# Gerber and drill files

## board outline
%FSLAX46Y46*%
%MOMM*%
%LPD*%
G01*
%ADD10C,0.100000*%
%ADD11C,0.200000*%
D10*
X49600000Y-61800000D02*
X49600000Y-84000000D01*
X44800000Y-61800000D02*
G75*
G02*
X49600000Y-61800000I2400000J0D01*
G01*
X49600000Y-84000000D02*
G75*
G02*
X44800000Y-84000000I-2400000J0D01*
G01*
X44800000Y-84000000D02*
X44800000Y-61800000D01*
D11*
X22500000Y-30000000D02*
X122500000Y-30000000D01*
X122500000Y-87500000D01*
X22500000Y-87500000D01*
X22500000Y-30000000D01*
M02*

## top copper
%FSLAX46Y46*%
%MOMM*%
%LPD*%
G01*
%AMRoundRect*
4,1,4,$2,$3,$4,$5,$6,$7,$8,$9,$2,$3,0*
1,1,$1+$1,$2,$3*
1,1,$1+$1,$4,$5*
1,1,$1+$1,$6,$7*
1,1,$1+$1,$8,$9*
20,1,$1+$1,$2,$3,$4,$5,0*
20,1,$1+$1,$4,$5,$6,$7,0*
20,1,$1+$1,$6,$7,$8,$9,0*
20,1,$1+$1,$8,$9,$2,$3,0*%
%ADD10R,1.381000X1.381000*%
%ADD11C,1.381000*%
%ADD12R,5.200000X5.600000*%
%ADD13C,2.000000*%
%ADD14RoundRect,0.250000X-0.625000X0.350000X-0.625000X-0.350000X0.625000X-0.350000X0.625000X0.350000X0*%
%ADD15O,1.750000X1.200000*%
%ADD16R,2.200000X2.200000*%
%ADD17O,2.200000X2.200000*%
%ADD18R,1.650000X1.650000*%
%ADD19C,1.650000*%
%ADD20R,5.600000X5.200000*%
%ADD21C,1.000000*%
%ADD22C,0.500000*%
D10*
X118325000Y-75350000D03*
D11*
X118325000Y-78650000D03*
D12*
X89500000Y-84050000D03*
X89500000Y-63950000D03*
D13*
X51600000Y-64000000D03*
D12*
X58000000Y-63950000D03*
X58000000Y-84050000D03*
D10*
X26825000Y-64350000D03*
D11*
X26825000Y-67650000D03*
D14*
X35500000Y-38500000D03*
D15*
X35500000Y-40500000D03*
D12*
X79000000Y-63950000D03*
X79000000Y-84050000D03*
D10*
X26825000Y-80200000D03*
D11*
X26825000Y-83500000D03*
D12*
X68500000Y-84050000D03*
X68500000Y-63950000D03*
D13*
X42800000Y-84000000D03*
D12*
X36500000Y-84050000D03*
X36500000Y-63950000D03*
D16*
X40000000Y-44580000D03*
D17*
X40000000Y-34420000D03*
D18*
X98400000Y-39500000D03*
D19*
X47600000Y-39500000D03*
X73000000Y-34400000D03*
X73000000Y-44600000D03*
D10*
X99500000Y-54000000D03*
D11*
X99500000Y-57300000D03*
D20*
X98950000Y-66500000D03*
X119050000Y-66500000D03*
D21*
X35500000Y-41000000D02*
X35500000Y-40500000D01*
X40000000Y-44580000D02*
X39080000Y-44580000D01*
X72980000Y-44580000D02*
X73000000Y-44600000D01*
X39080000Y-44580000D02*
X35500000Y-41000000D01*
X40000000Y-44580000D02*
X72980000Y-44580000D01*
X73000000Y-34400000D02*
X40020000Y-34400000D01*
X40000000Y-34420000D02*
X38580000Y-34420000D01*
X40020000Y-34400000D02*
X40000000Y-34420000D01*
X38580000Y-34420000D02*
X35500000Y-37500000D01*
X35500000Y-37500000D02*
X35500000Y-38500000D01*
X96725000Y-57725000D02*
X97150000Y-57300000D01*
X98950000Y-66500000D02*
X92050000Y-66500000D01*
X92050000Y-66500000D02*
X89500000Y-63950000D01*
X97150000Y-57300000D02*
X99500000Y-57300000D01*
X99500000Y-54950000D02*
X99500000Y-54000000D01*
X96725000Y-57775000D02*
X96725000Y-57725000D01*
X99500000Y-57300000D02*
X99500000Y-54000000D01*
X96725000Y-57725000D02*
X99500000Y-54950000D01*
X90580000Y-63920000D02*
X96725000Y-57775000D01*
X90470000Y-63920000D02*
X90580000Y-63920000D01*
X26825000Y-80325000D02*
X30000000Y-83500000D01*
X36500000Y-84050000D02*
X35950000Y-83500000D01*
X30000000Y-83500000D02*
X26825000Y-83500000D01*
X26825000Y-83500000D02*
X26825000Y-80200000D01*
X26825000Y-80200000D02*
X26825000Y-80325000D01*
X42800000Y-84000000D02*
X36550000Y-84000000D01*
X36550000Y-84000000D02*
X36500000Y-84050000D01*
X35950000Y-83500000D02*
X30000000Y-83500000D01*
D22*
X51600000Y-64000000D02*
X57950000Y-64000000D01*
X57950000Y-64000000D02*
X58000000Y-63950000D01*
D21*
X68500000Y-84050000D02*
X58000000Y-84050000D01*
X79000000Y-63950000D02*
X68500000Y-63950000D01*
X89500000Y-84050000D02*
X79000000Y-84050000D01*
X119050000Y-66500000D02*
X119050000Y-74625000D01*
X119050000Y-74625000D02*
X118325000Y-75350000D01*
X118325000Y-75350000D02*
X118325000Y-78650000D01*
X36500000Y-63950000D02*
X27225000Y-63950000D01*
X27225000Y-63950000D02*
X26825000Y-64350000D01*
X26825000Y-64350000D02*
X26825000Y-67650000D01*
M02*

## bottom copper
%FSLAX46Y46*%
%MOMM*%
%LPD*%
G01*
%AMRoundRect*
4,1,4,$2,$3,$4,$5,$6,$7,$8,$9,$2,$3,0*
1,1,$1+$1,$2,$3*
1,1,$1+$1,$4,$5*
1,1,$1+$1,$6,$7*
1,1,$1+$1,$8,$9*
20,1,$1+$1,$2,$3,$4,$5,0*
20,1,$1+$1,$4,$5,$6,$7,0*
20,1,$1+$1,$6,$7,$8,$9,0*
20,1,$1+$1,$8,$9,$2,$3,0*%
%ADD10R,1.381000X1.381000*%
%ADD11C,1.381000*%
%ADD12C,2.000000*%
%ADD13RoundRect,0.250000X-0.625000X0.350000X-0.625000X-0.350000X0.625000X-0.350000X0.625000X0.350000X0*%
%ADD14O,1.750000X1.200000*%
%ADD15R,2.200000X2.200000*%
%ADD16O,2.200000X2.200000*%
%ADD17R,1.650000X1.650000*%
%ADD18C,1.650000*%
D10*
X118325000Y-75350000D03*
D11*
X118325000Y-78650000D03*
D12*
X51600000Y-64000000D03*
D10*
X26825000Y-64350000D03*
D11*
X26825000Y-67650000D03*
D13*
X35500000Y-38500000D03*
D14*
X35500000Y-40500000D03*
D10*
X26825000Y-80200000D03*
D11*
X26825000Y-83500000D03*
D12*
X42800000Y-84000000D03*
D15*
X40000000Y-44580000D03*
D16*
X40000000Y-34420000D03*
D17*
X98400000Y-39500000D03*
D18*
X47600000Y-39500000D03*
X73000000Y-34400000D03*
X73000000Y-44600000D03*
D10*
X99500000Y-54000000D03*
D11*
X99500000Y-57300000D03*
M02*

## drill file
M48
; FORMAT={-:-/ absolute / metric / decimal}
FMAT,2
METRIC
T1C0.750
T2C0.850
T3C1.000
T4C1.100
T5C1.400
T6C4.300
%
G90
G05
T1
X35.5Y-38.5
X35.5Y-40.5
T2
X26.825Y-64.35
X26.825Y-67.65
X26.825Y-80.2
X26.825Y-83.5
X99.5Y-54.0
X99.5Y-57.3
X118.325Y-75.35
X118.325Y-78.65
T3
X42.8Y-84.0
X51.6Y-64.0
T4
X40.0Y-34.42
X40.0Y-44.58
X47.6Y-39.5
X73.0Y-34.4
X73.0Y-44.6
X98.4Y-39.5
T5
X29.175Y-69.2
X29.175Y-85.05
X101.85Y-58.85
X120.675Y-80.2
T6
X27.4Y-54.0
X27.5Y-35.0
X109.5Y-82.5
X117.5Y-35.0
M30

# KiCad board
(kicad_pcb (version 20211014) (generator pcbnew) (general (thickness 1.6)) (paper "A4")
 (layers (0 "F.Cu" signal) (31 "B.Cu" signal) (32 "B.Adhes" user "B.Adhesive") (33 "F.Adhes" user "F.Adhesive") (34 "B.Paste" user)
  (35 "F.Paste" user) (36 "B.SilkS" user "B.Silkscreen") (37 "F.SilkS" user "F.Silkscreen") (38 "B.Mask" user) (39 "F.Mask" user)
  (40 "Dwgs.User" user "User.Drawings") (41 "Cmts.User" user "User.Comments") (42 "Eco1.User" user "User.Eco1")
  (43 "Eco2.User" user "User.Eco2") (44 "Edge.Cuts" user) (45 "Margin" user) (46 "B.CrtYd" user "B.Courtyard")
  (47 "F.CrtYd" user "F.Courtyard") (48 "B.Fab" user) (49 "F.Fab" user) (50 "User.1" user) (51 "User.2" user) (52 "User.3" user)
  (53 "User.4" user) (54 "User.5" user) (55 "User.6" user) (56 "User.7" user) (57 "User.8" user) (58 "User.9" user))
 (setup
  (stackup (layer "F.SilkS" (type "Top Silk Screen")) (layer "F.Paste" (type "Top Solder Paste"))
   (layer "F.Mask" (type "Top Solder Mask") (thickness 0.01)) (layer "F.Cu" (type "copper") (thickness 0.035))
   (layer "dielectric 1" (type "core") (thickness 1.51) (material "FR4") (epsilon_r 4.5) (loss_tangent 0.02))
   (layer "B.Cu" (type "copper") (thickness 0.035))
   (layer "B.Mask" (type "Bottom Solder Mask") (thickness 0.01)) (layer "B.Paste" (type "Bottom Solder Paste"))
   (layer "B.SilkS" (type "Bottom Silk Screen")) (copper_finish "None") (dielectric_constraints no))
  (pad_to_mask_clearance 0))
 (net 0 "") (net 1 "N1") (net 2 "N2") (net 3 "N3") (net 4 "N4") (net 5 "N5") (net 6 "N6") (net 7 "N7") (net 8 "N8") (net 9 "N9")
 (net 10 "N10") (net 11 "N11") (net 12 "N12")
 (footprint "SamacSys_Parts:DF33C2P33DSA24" (layer "F.Cu") (at 118.325 75.35 -90)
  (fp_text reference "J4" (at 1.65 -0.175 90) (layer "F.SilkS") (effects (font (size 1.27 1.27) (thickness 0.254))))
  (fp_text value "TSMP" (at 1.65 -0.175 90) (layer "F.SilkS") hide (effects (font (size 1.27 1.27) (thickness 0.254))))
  (pad "" np_thru_hole circle locked (at 4.85 -2.35 270) (size 1.4 1.4) (drill 1.4) (layers *.Cu *.Mask))
  (pad "1" thru_hole rect locked (at 0 0 270) (size 1.381 1.381) (drill 0.85) (layers *.Cu *.Mask) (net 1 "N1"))
  (pad "2" thru_hole circle locked (at 3.3 0 270) (size 1.381 1.381) (drill 0.85) (layers *.Cu *.Mask) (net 1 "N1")))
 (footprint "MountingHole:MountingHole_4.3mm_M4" (layer "F.Cu") (at 117.5 35 180)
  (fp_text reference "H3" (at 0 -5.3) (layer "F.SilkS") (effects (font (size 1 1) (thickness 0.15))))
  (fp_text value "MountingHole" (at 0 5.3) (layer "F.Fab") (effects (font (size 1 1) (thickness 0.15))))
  (pad "" np_thru_hole circle (at 0 0 180) (size 4.3 4.3) (drill 4.3) (layers *.Cu *.Mask)))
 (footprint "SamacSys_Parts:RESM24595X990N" (layer "F.Cu") (at 89.5 74 90)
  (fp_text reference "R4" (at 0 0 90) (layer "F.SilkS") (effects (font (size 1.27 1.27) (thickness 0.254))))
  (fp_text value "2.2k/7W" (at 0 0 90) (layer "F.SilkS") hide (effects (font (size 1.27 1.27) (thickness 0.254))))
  (pad "1" smd rect locked (at -10.05 0 180) (size 5.2 5.6) (layers "F.Cu" "F.Paste" "F.Mask") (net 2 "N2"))
  (pad "2" smd rect locked (at 10.05 0 180) (size 5.2 5.6) (layers "F.Cu" "F.Paste" "F.Mask") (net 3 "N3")))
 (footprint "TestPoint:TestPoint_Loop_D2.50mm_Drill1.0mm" (layer "F.Cu") (at 51.6 64)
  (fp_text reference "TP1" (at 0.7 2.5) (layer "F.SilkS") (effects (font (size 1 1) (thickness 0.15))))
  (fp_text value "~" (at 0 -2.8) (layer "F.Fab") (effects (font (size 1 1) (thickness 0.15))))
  (pad "1" thru_hole circle (at 0 0) (size 2 2) (drill 1) (layers *.Cu *.Mask) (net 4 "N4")))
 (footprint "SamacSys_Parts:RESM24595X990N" (layer "F.Cu") (at 58 74 -90)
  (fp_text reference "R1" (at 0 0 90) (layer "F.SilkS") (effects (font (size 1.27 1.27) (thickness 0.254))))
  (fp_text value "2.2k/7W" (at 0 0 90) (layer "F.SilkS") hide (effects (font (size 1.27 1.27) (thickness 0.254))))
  (pad "1" smd rect locked (at -10.05 0) (size 5.2 5.6) (layers "F.Cu" "F.Paste" "F.Mask") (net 4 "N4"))
  (pad "2" smd rect locked (at 10.05 0) (size 5.2 5.6) (layers "F.Cu" "F.Paste" "F.Mask") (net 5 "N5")))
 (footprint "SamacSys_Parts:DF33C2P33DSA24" (layer "F.Cu") (at 26.825 64.35 -90)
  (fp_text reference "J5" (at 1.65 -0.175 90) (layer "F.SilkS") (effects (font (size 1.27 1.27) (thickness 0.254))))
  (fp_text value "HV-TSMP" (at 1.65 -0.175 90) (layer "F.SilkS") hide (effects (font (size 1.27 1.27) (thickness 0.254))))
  (pad "" np_thru_hole circle locked (at 4.85 -2.35 270) (size 1.4 1.4) (drill 1.4) (layers *.Cu *.Mask))
  (pad "1" thru_hole rect locked (at 0 0 270) (size 1.381 1.381) (drill 0.85) (layers *.Cu *.Mask) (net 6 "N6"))
  (pad "2" thru_hole circle locked (at 3.3 0 270) (size 1.381 1.381) (drill 0.85) (layers *.Cu *.Mask) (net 6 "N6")))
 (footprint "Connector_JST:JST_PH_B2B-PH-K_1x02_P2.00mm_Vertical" (layer "F.Cu") (at 35.5 38.5 -90)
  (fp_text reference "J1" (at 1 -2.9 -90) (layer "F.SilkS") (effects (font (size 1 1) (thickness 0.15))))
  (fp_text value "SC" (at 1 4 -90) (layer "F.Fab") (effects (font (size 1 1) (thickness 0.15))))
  (pad "1" thru_hole roundrect (at 0 0 270) (size 1.2 1.75) (drill 0.75) (layers *.Cu *.Mask) (roundrect_rratio 0.2083333333) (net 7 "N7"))
  (pad "2" thru_hole oval (at 2 0 270) (size 1.2 1.75) (drill 0.75) (layers *.Cu *.Mask) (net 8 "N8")))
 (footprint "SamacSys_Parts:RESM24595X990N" (layer "F.Cu") (at 79 74 -90)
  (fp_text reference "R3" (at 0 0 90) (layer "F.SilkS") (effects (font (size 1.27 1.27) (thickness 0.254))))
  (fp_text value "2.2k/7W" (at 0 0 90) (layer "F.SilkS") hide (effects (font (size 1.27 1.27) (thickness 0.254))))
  (pad "1" smd rect locked (at -10.05 0) (size 5.2 5.6) (layers "F.Cu" "F.Paste" "F.Mask") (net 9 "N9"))
  (pad "2" smd rect locked (at 10.05 0) (size 5.2 5.6) (layers "F.Cu" "F.Paste" "F.Mask") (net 2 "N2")))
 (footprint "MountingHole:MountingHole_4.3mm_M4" (layer "F.Cu") (at 27.5 35 180)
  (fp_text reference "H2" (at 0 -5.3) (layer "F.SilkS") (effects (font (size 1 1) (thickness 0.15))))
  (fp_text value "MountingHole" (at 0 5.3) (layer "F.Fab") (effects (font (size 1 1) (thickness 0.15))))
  (pad "" np_thru_hole circle (at 0 0 180) (size 4.3 4.3) (drill 4.3) (layers *.Cu *.Mask)))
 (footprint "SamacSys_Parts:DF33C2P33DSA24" (layer "F.Cu") (at 26.825 80.2 -90)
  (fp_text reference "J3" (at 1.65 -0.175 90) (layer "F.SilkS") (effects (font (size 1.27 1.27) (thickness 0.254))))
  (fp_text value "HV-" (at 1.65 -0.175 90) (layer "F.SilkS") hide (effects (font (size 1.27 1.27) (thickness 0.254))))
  (pad "" np_thru_hole circle locked (at 4.85 -2.35 270) (size 1.4 1.4) (drill 1.4) (layers *.Cu *.Mask))
  (pad "1" thru_hole rect locked (at 0 0 270) (size 1.381 1.381) (drill 0.85) (layers *.Cu *.Mask) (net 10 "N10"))
  (pad "2" thru_hole circle locked (at 3.3 0 270) (size 1.381 1.381) (drill 0.85) (layers *.Cu *.Mask) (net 10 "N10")))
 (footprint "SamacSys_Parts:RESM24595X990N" (layer "F.Cu") (at 68.5 74 90)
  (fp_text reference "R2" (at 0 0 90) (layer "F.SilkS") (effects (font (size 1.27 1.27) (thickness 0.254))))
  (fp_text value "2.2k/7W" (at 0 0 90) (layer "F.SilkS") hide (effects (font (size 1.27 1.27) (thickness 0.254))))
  (pad "1" smd rect locked (at -10.05 0 180) (size 5.2 5.6) (layers "F.Cu" "F.Paste" "F.Mask") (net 5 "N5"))
  (pad "2" smd rect locked (at 10.05 0 180) (size 5.2 5.6) (layers "F.Cu" "F.Paste" "F.Mask") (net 9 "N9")))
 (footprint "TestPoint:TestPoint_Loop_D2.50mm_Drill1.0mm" (layer "F.Cu") (at 42.8 84 -90)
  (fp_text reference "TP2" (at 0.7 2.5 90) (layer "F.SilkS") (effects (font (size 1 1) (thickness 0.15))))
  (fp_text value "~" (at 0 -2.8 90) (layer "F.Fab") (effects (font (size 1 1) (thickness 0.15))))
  (pad "1" thru_hole circle (at 0 0 270) (size 2 2) (drill 1) (layers *.Cu *.Mask) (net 10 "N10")))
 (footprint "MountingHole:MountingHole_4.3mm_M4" (layer "F.Cu") (at 109.5 82.5)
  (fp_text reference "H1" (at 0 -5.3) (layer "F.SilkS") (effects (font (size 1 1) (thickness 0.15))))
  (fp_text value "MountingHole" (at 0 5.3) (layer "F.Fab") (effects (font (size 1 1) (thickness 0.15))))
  (pad "" np_thru_hole circle (at 0 0) (size 4.3 4.3) (drill 4.3) (layers *.Cu *.Mask)))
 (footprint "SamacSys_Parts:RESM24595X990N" (layer "F.Cu") (at 36.5 74 90)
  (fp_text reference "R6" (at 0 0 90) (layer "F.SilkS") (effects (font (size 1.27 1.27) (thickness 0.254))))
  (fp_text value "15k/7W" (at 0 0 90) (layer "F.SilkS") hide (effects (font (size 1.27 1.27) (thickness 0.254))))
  (pad "1" smd rect locked (at -10.05 0 180) (size 5.2 5.6) (layers "F.Cu" "F.Paste" "F.Mask") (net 10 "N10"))
  (pad "2" smd rect locked (at 10.05 0 180) (size 5.2 5.6) (layers "F.Cu" "F.Paste" "F.Mask") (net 6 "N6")))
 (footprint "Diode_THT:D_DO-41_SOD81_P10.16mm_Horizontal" (layer "F.Cu") (at 40 44.58 90)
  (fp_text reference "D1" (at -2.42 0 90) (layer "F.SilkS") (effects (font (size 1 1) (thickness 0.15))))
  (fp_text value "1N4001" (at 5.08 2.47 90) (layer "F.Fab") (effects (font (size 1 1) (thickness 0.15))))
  (pad "1" thru_hole rect (at 0 0 90) (size 2.2 2.2) (drill 1.1) (layers *.Cu *.Mask) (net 8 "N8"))
  (pad "2" thru_hole oval (at 10.16 0 90) (size 2.2 2.2) (drill 1.1) (layers *.Cu *.Mask) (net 7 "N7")))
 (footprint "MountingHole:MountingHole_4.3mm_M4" (layer "F.Cu") (at 27.4 54)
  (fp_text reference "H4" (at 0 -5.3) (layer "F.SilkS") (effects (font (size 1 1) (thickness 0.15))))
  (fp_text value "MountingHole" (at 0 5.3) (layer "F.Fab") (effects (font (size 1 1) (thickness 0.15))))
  (pad "" np_thru_hole circle (at 0 0) (size 4.3 4.3) (drill 4.3) (layers *.Cu *.Mask)))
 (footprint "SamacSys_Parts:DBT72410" (layer "F.Cu") (at 98.4 39.5 180)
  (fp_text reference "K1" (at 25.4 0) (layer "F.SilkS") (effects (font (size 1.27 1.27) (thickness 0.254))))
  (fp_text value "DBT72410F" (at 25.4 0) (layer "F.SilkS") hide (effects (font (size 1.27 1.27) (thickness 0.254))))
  (pad "1" thru_hole rect (at 0 0 180) (size 1.65 1.65) (drill 1.1) (layers *.Cu *.Mask) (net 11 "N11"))
  (pad "2" thru_hole circle (at 50.8 0 180) (size 1.65 1.65) (drill 1.1) (layers *.Cu *.Mask) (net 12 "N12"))
  (pad "3" thru_hole circle (at 25.4 5.1 180) (size 1.65 1.65) (drill 1.1) (layers *.Cu *.Mask) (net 7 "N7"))
  (pad "4" thru_hole circle (at 25.4 -5.1 180) (size 1.65 1.65) (drill 1.1) (layers *.Cu *.Mask) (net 8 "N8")))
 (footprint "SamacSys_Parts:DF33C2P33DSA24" (layer "F.Cu") (at 99.5 54 -90)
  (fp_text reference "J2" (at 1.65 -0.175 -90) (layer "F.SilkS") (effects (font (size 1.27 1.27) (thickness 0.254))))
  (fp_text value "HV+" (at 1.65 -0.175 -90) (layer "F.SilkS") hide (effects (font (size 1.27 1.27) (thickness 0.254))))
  (pad "" np_thru_hole circle locked (at 4.85 -2.35 270) (size 1.4 1.4) (drill 1.4) (layers *.Cu *.Mask))
  (pad "1" thru_hole rect locked (at 0 0 270) (size 1.381 1.381) (drill 0.85) (layers *.Cu *.Mask) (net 3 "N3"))
  (pad "2" thru_hole circle locked (at 3.3 0 270) (size 1.381 1.381) (drill 0.85) (layers *.Cu *.Mask) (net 3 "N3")))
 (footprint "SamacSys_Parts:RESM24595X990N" (layer "F.Cu") (at 109 66.5)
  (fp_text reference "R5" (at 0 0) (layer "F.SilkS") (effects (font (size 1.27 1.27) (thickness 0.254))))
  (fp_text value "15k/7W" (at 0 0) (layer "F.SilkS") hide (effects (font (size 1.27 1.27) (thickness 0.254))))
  (pad "1" smd rect locked (at -10.05 0 90) (size 5.2 5.6) (layers "F.Cu" "F.Paste" "F.Mask") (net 3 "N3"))
  (pad "2" smd rect locked (at 10.05 0 90) (size 5.2 5.6) (layers "F.Cu" "F.Paste" "F.Mask") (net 1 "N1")))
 (gr_line (start 49.6 61.8) (end 49.6 84) (layer "Edge.Cuts") (width 0.1))
 (gr_arc (start 44.8 61.8) (mid 47.2 59.4) (end 49.6 61.8) (layer "Edge.Cuts") (width 0.1))
 (gr_arc (start 49.6 84) (mid 47.2 86.4) (end 44.8 84) (layer "Edge.Cuts") (width 0.1))
 (gr_line (start 44.8 84) (end 44.8 61.8) (layer "Edge.Cuts") (width 0.1))
 (gr_rect (start 122.5 87.5) (end 22.5 30) (layer "Edge.Cuts") (width 0.2) (fill none))
 (segment (start 35.5 41) (end 35.5 40.5) (width 1) (layer "F.Cu") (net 8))
 (segment (start 40 44.58) (end 39.08 44.58) (width 1) (layer "F.Cu") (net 8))
 (segment (start 72.98 44.58) (end 73 44.6) (width 1) (layer "F.Cu") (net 8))
 (segment (start 39.08 44.58) (end 35.5 41) (width 1) (layer "F.Cu") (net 8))
 (segment (start 40 44.58) (end 72.98 44.58) (width 1) (layer "F.Cu") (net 8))
 (segment (start 73 34.4) (end 40.02 34.4) (width 1) (layer "F.Cu") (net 7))
 (segment (start 40 34.42) (end 38.58 34.42) (width 1) (layer "F.Cu") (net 7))
 (segment (start 40.02 34.4) (end 40 34.42) (width 1) (layer "F.Cu") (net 7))
 (segment (start 38.58 34.42) (end 35.5 37.5) (width 1) (layer "F.Cu") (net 7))
 (segment (start 35.5 37.5) (end 35.5 38.5) (width 1) (layer "F.Cu") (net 7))
 (segment (start 96.725 57.725) (end 97.15 57.3) (width 1) (layer "F.Cu") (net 3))
 (segment (start 98.95 66.5) (end 92.05 66.5) (width 1) (layer "F.Cu") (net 3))
 (segment (start 92.05 66.5) (end 89.5 63.95) (width 1) (layer "F.Cu") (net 3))
 (segment (start 97.15 57.3) (end 99.5 57.3) (width 1) (layer "F.Cu") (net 3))
 (segment (start 99.5 54.95) (end 99.5 54) (width 1) (layer "F.Cu") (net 3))
 (segment (start 96.725 57.775) (end 96.725 57.725) (width 1) (layer "F.Cu") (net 3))
 (segment (start 99.5 57.3) (end 99.5 54) (width 1) (layer "F.Cu") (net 3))
 (segment (start 96.725 57.725) (end 99.5 54.95) (width 1) (layer "F.Cu") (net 3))
 (segment (start 90.58 63.92) (end 96.725 57.775) (width 1) (layer "F.Cu") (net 3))
 (segment (start 90.47 63.92) (end 90.58 63.92) (width 1) (layer "F.Cu") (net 3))
 (segment (start 26.825 80.325) (end 30 83.5) (width 1) (layer "F.Cu") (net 10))
 (segment (start 36.5 84.05) (end 35.95 83.5) (width 1) (layer "F.Cu") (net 10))
 (segment (start 30 83.5) (end 26.825 83.5) (width 1) (layer "F.Cu") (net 10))
 (segment (start 26.825 83.5) (end 26.825 80.2) (width 1) (layer "F.Cu") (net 10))
 (segment (start 26.825 80.2) (end 26.825 80.325) (width 1) (layer "F.Cu") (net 10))
 (segment (start 42.8 84) (end 36.55 84) (width 1) (layer "F.Cu") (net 10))
 (segment (start 36.55 84) (end 36.5 84.05) (width 1) (layer "F.Cu") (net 10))
 (segment (start 35.95 83.5) (end 30 83.5) (width 1) (layer "F.Cu") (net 10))
 (segment (start 51.6 64) (end 57.95 64) (width 0.5) (layer "F.Cu") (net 4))
 (segment (start 57.95 64) (end 58 63.95) (width 0.5) (layer "F.Cu") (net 4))
 (segment (start 68.5 84.05) (end 58 84.05) (width 1) (layer "F.Cu") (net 5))
 (segment (start 79 63.95) (end 68.5 63.95) (width 1) (layer "F.Cu") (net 9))
 (segment (start 89.5 84.05) (end 79 84.05) (width 1) (layer "F.Cu") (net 2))
 (segment (start 119.05 66.5) (end 119.05 74.625) (width 1) (layer "F.Cu") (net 1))
 (segment (start 119.05 74.625) (end 118.325 75.35) (width 1) (layer "F.Cu") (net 1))
 (segment (start 118.325 75.35) (end 118.325 78.65) (width 1) (layer "F.Cu") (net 1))
 (segment (start 36.5 63.95) (end 27.225 63.95) (width 1) (layer "F.Cu") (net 6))
 (segment (start 27.225 63.95) (end 26.825 64.35) (width 1) (layer "F.Cu") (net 6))
 (segment (start 26.825 64.35) (end 26.825 67.65) (width 1) (layer "F.Cu") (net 6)))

